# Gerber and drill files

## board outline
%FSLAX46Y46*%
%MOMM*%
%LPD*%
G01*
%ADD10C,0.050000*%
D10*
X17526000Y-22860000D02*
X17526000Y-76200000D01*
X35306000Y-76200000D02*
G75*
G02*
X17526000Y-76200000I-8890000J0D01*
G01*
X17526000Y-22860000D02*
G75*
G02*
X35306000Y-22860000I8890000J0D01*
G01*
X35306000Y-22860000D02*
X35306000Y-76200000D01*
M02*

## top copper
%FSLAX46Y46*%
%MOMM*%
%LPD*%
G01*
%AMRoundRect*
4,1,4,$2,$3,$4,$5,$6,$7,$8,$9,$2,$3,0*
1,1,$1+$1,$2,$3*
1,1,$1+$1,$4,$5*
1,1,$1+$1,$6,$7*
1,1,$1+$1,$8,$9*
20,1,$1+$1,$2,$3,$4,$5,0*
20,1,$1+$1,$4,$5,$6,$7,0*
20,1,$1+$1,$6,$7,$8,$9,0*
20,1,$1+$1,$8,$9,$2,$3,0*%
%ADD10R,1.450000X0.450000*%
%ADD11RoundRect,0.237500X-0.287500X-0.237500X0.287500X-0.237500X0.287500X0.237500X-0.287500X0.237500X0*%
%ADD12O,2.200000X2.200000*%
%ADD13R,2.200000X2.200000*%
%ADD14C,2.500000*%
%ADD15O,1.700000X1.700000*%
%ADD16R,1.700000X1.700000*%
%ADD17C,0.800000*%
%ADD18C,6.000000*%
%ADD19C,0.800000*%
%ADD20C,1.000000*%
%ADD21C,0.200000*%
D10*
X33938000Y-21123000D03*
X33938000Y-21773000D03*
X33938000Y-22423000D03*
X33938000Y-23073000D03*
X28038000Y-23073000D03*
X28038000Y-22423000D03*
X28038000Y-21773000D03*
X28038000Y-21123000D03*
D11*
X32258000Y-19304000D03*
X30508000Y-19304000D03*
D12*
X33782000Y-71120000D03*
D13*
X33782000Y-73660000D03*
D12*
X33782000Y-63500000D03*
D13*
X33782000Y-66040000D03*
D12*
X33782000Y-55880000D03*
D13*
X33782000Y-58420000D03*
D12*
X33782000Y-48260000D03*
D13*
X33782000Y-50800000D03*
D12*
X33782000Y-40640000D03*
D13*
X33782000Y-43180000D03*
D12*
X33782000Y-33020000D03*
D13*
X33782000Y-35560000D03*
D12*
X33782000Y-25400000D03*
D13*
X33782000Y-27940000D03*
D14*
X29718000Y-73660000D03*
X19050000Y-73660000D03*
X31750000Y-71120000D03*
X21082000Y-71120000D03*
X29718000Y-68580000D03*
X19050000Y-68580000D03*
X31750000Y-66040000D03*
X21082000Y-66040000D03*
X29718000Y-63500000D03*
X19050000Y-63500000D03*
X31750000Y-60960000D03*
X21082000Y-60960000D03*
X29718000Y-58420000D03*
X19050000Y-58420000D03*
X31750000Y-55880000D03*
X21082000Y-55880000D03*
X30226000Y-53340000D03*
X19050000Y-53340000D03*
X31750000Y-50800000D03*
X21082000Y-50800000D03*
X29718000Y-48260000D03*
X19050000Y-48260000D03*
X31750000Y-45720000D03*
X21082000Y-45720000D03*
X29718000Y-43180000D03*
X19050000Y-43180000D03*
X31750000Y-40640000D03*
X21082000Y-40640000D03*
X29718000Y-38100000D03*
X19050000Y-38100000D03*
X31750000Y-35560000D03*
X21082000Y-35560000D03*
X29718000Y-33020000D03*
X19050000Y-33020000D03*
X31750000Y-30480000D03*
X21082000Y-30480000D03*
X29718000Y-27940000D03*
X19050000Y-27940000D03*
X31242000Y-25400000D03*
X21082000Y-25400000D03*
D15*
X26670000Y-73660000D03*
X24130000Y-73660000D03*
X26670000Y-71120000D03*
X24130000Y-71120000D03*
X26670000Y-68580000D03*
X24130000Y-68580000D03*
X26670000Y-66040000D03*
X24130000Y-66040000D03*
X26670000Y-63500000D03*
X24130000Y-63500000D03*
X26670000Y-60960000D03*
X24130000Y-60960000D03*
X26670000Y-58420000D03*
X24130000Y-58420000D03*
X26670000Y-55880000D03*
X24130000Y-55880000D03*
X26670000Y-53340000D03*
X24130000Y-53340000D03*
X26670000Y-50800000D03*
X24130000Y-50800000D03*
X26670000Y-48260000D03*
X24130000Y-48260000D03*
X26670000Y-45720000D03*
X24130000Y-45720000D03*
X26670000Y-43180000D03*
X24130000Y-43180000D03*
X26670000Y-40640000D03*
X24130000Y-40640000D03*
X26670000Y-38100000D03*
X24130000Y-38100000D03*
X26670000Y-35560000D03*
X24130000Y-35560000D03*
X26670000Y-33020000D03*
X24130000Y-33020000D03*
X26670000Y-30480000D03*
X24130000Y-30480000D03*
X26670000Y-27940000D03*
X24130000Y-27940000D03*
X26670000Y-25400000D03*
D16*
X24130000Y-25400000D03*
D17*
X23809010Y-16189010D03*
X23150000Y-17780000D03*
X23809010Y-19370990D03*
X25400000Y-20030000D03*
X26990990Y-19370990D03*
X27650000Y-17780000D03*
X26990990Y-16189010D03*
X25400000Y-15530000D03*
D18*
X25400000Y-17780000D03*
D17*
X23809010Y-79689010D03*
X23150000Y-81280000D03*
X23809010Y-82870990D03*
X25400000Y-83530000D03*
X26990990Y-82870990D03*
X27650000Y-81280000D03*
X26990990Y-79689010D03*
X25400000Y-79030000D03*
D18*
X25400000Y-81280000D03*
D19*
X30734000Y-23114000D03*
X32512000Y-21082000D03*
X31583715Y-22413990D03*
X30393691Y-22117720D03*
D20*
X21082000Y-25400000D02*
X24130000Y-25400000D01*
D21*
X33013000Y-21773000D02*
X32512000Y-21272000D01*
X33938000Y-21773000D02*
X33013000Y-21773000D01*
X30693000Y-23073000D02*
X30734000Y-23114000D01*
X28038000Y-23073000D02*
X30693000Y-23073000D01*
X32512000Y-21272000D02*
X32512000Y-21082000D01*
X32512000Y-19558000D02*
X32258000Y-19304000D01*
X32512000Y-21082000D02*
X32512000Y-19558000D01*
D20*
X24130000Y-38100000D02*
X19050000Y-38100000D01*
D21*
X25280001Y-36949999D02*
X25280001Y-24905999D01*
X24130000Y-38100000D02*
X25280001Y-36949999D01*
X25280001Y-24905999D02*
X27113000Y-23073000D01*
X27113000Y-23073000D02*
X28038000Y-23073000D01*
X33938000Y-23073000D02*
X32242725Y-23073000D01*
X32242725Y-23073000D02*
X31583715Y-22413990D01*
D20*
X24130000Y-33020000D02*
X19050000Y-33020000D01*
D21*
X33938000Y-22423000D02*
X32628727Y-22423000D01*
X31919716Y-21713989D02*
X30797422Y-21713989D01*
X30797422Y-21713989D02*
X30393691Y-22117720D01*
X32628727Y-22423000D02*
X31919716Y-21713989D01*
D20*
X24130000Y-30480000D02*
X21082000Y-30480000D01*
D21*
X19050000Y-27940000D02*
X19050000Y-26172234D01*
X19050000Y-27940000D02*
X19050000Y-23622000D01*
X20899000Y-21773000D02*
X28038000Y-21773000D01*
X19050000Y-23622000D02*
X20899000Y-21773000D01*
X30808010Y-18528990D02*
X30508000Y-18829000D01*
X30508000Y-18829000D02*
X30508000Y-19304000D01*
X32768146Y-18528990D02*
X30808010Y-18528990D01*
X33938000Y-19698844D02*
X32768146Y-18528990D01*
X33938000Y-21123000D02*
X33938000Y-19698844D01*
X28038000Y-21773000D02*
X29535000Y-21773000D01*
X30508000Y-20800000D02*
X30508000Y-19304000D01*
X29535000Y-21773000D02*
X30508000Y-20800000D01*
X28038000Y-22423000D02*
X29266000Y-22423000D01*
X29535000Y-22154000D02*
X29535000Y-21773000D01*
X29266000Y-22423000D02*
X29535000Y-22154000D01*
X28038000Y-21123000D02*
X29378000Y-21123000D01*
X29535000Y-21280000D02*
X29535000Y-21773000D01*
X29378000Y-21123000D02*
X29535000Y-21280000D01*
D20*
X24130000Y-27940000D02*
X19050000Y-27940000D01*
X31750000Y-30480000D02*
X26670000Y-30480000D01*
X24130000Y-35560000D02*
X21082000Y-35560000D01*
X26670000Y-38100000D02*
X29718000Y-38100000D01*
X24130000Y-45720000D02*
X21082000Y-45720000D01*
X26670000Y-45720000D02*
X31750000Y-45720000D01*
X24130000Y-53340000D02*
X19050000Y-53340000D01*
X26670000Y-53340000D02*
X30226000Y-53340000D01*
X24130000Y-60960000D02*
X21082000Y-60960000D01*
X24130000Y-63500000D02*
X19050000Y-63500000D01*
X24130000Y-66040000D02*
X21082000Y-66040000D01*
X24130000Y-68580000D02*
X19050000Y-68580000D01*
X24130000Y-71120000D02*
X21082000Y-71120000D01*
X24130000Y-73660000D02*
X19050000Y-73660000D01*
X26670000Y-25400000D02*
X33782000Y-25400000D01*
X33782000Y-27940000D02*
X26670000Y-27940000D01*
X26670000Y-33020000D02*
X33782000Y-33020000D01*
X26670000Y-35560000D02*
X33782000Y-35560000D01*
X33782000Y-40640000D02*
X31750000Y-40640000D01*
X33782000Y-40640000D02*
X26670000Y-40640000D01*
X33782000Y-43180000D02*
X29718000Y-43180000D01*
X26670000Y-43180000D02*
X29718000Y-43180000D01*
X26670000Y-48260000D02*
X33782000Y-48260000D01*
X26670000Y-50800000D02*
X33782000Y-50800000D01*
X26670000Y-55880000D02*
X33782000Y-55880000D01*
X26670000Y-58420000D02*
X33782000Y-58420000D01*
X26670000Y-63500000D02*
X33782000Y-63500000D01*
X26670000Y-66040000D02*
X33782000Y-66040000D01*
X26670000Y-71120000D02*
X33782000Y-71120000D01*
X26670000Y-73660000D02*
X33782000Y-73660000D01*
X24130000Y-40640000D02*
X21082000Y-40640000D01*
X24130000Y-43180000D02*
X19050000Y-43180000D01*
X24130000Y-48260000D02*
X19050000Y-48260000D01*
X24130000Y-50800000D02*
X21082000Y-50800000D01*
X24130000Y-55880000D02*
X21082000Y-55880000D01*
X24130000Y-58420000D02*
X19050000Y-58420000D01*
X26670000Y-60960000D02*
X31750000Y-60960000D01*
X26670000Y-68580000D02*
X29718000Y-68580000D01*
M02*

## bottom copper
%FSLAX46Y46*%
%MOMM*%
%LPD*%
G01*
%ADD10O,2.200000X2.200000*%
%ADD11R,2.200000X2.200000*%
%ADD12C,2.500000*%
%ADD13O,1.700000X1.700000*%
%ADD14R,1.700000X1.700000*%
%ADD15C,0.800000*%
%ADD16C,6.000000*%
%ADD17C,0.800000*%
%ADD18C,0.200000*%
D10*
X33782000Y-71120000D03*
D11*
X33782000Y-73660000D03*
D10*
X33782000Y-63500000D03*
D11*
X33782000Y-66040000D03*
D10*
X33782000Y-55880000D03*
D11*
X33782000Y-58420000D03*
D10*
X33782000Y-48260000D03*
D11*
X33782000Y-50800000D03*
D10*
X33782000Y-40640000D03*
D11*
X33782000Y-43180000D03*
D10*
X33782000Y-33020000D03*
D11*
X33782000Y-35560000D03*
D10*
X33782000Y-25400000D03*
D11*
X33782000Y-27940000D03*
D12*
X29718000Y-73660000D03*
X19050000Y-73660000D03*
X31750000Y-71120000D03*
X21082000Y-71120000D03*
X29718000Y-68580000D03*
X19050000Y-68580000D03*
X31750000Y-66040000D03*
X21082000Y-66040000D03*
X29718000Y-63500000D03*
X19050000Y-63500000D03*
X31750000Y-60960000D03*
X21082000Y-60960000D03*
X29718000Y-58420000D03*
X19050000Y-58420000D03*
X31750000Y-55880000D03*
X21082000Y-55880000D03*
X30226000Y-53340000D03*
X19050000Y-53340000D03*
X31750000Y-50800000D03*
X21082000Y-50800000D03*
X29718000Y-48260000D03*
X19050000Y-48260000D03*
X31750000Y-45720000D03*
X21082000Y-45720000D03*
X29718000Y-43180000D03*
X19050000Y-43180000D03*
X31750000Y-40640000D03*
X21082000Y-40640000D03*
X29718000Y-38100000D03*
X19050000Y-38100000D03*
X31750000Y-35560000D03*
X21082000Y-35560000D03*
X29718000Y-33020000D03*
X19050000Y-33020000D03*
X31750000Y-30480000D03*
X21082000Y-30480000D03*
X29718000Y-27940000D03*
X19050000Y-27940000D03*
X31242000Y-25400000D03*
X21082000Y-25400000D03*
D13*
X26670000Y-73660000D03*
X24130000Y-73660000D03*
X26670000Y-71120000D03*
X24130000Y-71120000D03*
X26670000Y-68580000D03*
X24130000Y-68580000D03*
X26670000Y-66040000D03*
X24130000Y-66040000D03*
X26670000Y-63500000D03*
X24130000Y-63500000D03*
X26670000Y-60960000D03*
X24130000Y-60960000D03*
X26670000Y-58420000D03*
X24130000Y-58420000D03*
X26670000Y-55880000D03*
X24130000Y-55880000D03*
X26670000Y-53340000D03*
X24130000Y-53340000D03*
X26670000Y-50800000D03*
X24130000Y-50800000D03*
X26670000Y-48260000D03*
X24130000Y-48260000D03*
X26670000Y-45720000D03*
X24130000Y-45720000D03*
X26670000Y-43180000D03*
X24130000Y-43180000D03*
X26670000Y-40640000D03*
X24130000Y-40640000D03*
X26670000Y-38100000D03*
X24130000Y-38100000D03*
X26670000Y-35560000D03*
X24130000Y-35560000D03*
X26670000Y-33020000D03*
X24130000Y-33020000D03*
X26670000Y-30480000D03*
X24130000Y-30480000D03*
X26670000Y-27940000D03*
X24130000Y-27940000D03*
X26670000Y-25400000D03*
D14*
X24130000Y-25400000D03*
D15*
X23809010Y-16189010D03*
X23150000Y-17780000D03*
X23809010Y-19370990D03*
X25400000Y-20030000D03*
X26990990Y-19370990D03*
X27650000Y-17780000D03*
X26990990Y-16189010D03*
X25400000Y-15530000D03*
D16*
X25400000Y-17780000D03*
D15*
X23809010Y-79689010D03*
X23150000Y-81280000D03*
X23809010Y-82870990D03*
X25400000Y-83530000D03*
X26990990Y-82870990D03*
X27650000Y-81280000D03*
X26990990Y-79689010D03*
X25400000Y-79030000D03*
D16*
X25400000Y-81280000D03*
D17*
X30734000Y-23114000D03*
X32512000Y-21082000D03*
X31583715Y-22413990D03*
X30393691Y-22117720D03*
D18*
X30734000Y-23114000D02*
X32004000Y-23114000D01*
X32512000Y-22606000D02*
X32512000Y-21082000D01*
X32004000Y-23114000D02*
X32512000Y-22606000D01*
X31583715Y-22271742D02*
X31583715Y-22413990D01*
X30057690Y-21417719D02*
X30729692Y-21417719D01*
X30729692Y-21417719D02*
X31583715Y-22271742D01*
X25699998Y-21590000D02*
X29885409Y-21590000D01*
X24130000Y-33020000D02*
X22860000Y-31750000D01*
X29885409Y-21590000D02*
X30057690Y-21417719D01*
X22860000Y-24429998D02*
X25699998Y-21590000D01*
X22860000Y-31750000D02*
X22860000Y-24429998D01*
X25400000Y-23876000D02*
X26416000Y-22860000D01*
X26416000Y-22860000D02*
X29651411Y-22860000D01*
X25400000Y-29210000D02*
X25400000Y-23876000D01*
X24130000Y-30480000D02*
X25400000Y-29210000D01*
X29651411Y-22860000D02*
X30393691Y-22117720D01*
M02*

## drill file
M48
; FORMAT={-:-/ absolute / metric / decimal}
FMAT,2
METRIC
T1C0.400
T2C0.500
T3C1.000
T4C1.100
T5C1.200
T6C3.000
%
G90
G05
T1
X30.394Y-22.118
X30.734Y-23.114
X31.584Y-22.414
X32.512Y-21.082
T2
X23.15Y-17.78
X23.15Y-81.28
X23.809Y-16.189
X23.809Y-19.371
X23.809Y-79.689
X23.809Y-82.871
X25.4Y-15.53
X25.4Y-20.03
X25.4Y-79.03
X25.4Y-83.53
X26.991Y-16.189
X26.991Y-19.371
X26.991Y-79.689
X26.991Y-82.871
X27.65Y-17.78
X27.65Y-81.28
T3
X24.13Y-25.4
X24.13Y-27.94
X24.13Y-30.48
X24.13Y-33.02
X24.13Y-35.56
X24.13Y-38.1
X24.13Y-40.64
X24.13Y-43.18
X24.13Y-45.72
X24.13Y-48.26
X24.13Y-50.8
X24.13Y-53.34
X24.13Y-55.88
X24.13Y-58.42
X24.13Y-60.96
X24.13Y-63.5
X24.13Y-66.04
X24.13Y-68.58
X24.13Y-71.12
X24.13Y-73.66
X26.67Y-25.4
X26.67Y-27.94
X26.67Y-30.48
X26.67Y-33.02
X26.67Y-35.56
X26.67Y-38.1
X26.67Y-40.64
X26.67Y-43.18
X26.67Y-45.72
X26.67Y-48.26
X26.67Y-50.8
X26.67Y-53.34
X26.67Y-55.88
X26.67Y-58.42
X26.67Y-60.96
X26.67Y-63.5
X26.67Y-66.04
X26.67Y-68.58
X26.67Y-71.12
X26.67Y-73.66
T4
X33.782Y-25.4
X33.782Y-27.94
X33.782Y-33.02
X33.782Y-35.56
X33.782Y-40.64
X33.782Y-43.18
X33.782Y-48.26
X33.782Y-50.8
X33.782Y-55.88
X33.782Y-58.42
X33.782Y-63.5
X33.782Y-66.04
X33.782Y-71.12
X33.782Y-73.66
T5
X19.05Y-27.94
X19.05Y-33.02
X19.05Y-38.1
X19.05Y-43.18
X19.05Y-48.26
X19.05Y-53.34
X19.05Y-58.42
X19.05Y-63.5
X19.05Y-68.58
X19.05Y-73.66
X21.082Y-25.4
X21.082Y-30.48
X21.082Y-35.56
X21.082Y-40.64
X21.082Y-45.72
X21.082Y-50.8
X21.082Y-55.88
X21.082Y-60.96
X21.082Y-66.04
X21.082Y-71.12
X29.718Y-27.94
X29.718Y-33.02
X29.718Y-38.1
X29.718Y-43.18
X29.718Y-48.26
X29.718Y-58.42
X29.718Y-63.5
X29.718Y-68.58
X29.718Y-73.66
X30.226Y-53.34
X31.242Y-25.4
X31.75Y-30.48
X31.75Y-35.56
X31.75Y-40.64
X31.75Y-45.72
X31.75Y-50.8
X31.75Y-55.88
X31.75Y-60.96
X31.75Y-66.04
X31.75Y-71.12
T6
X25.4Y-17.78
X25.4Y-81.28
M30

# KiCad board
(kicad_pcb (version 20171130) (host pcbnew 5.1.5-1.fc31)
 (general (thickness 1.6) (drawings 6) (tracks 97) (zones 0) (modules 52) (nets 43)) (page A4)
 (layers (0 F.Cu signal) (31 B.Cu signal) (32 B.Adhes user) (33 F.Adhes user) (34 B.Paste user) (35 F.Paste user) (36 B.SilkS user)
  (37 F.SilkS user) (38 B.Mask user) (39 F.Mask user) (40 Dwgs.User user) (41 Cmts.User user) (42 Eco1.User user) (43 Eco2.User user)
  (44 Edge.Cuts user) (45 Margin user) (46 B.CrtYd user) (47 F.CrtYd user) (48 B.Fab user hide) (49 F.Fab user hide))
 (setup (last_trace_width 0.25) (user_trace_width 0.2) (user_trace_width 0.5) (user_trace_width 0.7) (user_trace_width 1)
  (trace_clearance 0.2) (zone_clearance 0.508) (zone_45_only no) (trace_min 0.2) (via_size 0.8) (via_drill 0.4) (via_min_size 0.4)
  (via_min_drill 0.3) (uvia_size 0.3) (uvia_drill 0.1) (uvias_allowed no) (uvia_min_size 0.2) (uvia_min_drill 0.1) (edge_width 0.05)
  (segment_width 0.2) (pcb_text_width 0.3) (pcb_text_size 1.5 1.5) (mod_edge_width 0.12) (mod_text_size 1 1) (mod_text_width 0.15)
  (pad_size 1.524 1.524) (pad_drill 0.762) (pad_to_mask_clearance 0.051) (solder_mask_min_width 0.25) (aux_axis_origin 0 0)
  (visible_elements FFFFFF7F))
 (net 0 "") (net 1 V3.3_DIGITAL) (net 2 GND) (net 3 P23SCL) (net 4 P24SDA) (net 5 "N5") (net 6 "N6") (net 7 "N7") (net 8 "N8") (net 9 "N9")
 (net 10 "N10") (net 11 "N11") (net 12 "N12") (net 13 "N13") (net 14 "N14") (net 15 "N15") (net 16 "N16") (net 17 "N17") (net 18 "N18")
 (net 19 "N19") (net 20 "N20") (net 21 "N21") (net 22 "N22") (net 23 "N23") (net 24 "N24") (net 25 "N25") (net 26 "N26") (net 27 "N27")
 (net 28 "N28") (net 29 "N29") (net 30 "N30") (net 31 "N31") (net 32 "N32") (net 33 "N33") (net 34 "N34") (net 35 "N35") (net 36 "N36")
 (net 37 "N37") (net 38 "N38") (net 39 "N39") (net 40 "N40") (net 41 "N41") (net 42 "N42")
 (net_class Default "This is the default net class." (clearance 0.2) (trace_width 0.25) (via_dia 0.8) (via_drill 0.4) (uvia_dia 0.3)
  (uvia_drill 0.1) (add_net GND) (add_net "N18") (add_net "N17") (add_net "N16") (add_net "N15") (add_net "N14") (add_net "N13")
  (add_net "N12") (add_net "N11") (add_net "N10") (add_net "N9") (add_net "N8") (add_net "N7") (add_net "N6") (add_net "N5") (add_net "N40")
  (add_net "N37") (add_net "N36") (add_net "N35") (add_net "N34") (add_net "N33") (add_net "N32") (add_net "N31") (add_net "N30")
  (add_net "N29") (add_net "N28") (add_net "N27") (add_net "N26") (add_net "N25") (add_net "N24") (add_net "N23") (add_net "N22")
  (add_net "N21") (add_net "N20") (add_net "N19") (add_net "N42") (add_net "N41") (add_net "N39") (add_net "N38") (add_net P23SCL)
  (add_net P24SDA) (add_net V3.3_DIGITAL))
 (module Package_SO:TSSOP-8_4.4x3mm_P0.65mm (layer F.Cu) (at 30.988 22.098)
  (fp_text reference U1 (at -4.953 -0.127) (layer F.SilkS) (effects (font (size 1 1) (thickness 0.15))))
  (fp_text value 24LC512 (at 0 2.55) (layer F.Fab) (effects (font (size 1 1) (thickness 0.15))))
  (pad 8 smd rect (at 2.95 -0.975) (size 1.45 0.45) (layers F.Cu F.Paste F.Mask) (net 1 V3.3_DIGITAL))
  (pad 7 smd rect (at 2.95 -0.325) (size 1.45 0.45) (layers F.Cu F.Paste F.Mask) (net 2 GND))
  (pad 6 smd rect (at 2.95 0.325) (size 1.45 0.45) (layers F.Cu F.Paste F.Mask) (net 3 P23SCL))
  (pad 5 smd rect (at 2.95 0.975) (size 1.45 0.45) (layers F.Cu F.Paste F.Mask) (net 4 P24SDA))
  (pad 4 smd rect (at -2.95 0.975) (size 1.45 0.45) (layers F.Cu F.Paste F.Mask) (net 2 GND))
  (pad 3 smd rect (at -2.95 0.325) (size 1.45 0.45) (layers F.Cu F.Paste F.Mask) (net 1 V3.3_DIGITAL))
  (pad 2 smd rect (at -2.95 -0.325) (size 1.45 0.45) (layers F.Cu F.Paste F.Mask) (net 1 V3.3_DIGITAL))
  (pad 1 smd rect (at -2.95 -0.975) (size 1.45 0.45) (layers F.Cu F.Paste F.Mask) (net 1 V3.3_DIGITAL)))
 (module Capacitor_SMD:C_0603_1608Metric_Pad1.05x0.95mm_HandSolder (layer F.Cu) (at 31.383 19.304)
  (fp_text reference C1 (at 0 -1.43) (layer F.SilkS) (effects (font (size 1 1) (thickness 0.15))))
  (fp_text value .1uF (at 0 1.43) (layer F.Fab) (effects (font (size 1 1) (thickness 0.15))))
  (pad 2 smd roundrect (at 0.875 0) (size 1.05 0.95) (layers F.Cu F.Paste F.Mask) (roundrect_rratio 0.25) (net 2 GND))
  (pad 1 smd roundrect (at -0.875 0) (size 1.05 0.95) (layers F.Cu F.Paste F.Mask) (roundrect_rratio 0.25) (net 1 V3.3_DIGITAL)))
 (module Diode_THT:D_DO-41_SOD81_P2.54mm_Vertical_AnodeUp (layer B.Cu) (at 33.782 73.66 90)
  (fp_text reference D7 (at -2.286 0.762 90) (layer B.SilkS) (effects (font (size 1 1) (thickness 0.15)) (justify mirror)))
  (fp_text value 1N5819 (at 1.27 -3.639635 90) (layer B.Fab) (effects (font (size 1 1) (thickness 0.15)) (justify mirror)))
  (pad 2 thru_hole oval (at 2.54 0 90) (size 2.2 2.2) (drill 1.1) (layers *.Cu *.Mask) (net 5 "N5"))
  (pad 1 thru_hole rect (at 0 0 90) (size 2.2 2.2) (drill 1.1) (layers *.Cu *.Mask) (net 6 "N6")))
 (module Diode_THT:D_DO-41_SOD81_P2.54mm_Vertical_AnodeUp (layer B.Cu) (at 33.782 66.04 90)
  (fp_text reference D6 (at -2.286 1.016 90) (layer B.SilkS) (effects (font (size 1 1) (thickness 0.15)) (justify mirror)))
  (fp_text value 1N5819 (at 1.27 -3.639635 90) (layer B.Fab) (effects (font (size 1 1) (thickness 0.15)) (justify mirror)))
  (pad 2 thru_hole oval (at 2.54 0 90) (size 2.2 2.2) (drill 1.1) (layers *.Cu *.Mask) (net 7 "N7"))
  (pad 1 thru_hole rect (at 0 0 90) (size 2.2 2.2) (drill 1.1) (layers *.Cu *.Mask) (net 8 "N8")))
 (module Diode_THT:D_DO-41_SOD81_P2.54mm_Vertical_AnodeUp (layer B.Cu) (at 33.782 58.42 90)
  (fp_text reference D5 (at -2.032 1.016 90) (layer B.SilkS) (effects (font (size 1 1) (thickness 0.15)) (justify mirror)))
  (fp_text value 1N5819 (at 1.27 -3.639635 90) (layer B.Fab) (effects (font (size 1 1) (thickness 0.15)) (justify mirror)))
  (pad 2 thru_hole oval (at 2.54 0 90) (size 2.2 2.2) (drill 1.1) (layers *.Cu *.Mask) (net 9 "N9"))
  (pad 1 thru_hole rect (at 0 0 90) (size 2.2 2.2) (drill 1.1) (layers *.Cu *.Mask) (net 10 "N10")))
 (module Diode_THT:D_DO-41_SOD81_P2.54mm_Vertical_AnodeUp (layer B.Cu) (at 33.782 50.8 90)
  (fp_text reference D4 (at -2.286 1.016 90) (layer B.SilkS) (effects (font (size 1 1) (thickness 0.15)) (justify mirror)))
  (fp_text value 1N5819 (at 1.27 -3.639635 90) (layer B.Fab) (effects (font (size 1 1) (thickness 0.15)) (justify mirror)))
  (pad 2 thru_hole oval (at 2.54 0 90) (size 2.2 2.2) (drill 1.1) (layers *.Cu *.Mask) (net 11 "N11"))
  (pad 1 thru_hole rect (at 0 0 90) (size 2.2 2.2) (drill 1.1) (layers *.Cu *.Mask) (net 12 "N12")))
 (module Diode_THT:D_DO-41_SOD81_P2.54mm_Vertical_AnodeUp (layer B.Cu) (at 33.782 43.18 90)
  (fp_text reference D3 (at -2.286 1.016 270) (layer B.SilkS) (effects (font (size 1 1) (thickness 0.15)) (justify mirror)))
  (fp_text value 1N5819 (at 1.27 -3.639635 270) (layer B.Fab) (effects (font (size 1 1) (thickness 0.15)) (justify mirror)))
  (pad 2 thru_hole oval (at 2.54 0 90) (size 2.2 2.2) (drill 1.1) (layers *.Cu *.Mask) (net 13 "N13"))
  (pad 1 thru_hole rect (at 0 0 90) (size 2.2 2.2) (drill 1.1) (layers *.Cu *.Mask) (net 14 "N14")))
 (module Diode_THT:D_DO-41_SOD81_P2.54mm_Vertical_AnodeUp (layer B.Cu) (at 33.782 35.56 90)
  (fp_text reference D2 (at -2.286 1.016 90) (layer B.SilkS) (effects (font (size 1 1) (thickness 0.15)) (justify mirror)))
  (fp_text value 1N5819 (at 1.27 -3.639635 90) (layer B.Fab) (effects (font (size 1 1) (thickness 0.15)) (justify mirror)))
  (pad 2 thru_hole oval (at 2.54 0 90) (size 2.2 2.2) (drill 1.1) (layers *.Cu *.Mask) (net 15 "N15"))
  (pad 1 thru_hole rect (at 0 0 90) (size 2.2 2.2) (drill 1.1) (layers *.Cu *.Mask) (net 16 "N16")))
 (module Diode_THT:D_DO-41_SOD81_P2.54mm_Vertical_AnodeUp (layer B.Cu) (at 33.782 27.94 90)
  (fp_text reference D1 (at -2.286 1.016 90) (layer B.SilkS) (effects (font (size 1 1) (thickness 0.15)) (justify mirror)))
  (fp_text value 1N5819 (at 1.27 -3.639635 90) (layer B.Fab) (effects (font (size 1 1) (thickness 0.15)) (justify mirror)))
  (pad 2 thru_hole oval (at 2.54 0 90) (size 2.2 2.2) (drill 1.1) (layers *.Cu *.Mask) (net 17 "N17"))
  (pad 1 thru_hole rect (at 0 0 90) (size 2.2 2.2) (drill 1.1) (layers *.Cu *.Mask) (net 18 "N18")))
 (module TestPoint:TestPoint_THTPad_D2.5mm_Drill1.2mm (layer F.Cu) (at 29.718 73.66 270)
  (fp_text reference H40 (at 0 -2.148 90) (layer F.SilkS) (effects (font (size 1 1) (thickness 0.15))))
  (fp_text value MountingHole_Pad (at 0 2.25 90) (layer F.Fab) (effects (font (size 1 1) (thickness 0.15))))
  (pad 1 thru_hole circle (at 0 0 270) (size 2.5 2.5) (drill 1.2) (layers *.Cu *.Mask) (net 6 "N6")))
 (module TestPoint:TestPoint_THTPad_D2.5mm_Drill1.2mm (layer F.Cu) (at 19.05 73.66 270)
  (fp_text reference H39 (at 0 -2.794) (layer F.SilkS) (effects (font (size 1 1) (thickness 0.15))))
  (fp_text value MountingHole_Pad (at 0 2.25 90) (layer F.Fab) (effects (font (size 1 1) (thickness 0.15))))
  (pad 1 thru_hole circle (at 0 0 270) (size 2.5 2.5) (drill 1.2) (layers *.Cu *.Mask) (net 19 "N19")))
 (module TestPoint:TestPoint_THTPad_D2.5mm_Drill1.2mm (layer F.Cu) (at 31.75 71.12 90)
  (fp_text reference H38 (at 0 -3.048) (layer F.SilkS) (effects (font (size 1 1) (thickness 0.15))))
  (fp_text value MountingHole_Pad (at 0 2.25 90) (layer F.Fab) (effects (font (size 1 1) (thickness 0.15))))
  (pad 1 thru_hole circle (at 0 0 90) (size 2.5 2.5) (drill 1.2) (layers *.Cu *.Mask) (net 5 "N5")))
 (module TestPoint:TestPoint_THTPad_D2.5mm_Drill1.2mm (layer F.Cu) (at 21.082 71.12 90)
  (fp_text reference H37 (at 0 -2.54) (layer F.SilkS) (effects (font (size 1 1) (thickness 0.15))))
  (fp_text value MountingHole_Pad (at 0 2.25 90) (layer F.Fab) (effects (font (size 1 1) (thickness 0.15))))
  (pad 1 thru_hole circle (at 0 0 90) (size 2.5 2.5) (drill 1.2) (layers *.Cu *.Mask) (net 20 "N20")))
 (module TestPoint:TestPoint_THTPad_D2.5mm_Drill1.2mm (layer F.Cu) (at 29.718 68.58 270)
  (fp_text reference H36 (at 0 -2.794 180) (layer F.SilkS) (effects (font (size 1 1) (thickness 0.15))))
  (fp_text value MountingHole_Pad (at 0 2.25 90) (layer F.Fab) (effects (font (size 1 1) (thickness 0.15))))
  (pad 1 thru_hole circle (at 0 0 270) (size 2.5 2.5) (drill 1.2) (layers *.Cu *.Mask) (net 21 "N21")))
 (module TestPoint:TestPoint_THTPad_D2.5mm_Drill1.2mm (layer F.Cu) (at 19.05 68.58 270)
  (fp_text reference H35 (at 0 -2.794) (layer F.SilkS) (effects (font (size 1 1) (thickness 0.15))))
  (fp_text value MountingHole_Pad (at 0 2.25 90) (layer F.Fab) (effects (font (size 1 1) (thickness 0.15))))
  (pad 1 thru_hole circle (at 0 0 270) (size 2.5 2.5) (drill 1.2) (layers *.Cu *.Mask) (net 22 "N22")))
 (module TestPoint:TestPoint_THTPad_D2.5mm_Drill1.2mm (layer F.Cu) (at 31.75 66.04 90)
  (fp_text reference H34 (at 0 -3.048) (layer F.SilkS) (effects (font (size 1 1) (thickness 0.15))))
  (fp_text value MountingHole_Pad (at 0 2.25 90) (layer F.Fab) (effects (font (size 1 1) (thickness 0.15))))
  (pad 1 thru_hole circle (at 0 0 90) (size 2.5 2.5) (drill 1.2) (layers *.Cu *.Mask) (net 8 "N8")))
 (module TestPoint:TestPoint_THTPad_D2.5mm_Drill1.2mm (layer F.Cu) (at 21.082 66.04 90)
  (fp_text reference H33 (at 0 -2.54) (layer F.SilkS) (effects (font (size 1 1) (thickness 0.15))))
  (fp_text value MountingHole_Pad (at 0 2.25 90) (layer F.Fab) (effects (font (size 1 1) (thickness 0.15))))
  (pad 1 thru_hole circle (at 0 0 90) (size 2.5 2.5) (drill 1.2) (layers *.Cu *.Mask) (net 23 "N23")))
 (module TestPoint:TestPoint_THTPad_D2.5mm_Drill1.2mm (layer F.Cu) (at 29.718 63.5 270)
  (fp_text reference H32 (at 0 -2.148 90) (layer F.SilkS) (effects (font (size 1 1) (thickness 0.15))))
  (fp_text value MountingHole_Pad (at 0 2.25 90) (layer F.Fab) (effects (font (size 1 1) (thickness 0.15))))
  (pad 1 thru_hole circle (at 0 0 270) (size 2.5 2.5) (drill 1.2) (layers *.Cu *.Mask) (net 7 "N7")))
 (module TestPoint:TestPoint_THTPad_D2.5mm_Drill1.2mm (layer F.Cu) (at 19.05 63.5 270)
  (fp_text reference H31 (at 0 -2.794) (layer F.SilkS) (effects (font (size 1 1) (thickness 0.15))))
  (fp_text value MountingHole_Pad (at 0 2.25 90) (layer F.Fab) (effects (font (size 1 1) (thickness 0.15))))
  (pad 1 thru_hole circle (at 0 0 270) (size 2.5 2.5) (drill 1.2) (layers *.Cu *.Mask) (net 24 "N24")))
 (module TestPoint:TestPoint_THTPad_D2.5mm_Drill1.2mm (layer F.Cu) (at 31.75 60.96 90)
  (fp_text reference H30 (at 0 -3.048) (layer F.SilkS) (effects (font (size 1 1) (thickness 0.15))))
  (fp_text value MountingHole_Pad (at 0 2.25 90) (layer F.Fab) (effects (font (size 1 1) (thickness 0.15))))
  (pad 1 thru_hole circle (at 0 0 90) (size 2.5 2.5) (drill 1.2) (layers *.Cu *.Mask) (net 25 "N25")))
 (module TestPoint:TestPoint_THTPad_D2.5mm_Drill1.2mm (layer F.Cu) (at 21.082 60.96 90)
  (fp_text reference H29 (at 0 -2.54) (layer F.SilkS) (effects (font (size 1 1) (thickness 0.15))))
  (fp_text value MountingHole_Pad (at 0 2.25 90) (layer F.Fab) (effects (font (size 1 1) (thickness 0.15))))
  (pad 1 thru_hole circle (at 0 0 90) (size 2.5 2.5) (drill 1.2) (layers *.Cu *.Mask) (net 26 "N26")))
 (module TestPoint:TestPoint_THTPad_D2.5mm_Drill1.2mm (layer F.Cu) (at 29.718 58.42 270)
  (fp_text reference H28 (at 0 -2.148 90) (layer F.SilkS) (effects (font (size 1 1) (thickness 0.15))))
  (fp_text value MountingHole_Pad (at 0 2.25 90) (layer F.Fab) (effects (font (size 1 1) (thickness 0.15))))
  (pad 1 thru_hole circle (at 0 0 270) (size 2.5 2.5) (drill 1.2) (layers *.Cu *.Mask) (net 10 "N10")))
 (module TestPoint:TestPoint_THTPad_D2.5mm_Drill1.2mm (layer F.Cu) (at 19.05 58.42 270)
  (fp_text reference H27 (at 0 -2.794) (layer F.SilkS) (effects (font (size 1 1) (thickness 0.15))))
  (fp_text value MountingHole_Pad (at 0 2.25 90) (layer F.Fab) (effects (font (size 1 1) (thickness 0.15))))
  (pad 1 thru_hole circle (at 0 0 270) (size 2.5 2.5) (drill 1.2) (layers *.Cu *.Mask) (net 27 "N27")))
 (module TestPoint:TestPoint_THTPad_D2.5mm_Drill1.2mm (layer F.Cu) (at 31.75 55.88 90)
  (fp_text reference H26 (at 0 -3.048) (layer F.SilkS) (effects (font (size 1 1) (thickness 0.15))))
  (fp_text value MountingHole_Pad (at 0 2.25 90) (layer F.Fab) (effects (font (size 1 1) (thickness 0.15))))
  (pad 1 thru_hole circle (at 0 0 90) (size 2.5 2.5) (drill 1.2) (layers *.Cu *.Mask) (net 9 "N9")))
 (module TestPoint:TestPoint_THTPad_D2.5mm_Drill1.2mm (layer F.Cu) (at 21.082 55.88 90)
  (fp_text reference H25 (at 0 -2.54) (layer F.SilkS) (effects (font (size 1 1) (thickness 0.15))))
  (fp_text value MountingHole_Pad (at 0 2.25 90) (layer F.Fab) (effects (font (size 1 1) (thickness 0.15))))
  (pad 1 thru_hole circle (at 0 0 90) (size 2.5 2.5) (drill 1.2) (layers *.Cu *.Mask) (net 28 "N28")))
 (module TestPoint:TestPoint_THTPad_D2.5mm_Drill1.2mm (layer F.Cu) (at 30.226 53.34 270)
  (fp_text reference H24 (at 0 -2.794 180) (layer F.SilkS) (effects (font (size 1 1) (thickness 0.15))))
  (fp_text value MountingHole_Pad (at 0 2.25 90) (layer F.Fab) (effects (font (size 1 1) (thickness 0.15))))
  (pad 1 thru_hole circle (at 0 0 270) (size 2.5 2.5) (drill 1.2) (layers *.Cu *.Mask) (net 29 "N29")))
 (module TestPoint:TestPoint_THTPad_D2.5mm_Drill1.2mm (layer F.Cu) (at 19.05 53.34 270)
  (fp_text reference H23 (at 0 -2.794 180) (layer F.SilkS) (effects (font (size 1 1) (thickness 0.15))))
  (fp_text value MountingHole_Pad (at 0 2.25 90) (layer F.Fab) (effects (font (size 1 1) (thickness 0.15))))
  (pad 1 thru_hole circle (at 0 0 270) (size 2.5 2.5) (drill 1.2) (layers *.Cu *.Mask) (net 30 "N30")))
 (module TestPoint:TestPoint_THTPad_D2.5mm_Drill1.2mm (layer F.Cu) (at 31.75 50.8 90)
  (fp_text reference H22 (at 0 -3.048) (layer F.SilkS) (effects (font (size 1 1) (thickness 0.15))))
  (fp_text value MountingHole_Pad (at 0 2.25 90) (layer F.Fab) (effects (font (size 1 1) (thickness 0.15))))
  (pad 1 thru_hole circle (at 0 0 90) (size 2.5 2.5) (drill 1.2) (layers *.Cu *.Mask) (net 12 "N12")))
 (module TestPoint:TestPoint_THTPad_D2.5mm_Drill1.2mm (layer F.Cu) (at 21.082 50.8 90)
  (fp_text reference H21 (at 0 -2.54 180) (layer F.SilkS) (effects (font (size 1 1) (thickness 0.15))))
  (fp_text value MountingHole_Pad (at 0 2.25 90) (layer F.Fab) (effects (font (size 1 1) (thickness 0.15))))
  (pad 1 thru_hole circle (at 0 0 90) (size 2.5 2.5) (drill 1.2) (layers *.Cu *.Mask) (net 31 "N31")))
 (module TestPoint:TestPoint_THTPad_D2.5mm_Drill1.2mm (layer F.Cu) (at 29.718 48.26 270)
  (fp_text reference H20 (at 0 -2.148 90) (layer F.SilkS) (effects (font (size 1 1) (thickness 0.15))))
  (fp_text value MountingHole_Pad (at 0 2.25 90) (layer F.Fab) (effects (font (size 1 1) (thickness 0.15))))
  (pad 1 thru_hole circle (at 0 0 270) (size 2.5 2.5) (drill 1.2) (layers *.Cu *.Mask) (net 11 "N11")))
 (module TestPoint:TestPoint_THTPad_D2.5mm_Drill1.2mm (layer F.Cu) (at 19.05 48.26 270)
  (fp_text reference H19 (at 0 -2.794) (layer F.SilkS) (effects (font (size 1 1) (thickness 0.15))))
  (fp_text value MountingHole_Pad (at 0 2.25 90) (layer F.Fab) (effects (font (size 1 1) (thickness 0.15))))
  (pad 1 thru_hole circle (at 0 0 270) (size 2.5 2.5) (drill 1.2) (layers *.Cu *.Mask) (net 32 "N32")))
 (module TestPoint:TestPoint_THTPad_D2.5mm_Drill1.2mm (layer F.Cu) (at 31.75 45.72 90)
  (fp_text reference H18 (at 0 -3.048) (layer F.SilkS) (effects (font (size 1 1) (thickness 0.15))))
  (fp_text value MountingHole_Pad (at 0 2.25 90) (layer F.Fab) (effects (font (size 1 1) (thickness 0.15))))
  (pad 1 thru_hole circle (at 0 0 90) (size 2.5 2.5) (drill 1.2) (layers *.Cu *.Mask) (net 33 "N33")))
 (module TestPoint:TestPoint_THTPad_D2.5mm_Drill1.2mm (layer F.Cu) (at 21.082 45.72 90)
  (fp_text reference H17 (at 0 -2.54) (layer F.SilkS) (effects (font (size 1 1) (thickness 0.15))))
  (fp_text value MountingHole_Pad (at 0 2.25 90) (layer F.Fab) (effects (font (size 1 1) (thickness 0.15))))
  (pad 1 thru_hole circle (at 0 0 90) (size 2.5 2.5) (drill 1.2) (layers *.Cu *.Mask) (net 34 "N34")))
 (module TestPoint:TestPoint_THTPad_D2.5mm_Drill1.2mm (layer F.Cu) (at 29.718 43.18 270)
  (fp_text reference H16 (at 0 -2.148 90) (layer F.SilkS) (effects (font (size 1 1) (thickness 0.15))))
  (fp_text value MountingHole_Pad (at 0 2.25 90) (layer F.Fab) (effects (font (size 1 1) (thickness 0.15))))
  (pad 1 thru_hole circle (at 0 0 270) (size 2.5 2.5) (drill 1.2) (layers *.Cu *.Mask) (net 14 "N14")))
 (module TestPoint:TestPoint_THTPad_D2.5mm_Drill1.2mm (layer F.Cu) (at 19.05 43.18 270)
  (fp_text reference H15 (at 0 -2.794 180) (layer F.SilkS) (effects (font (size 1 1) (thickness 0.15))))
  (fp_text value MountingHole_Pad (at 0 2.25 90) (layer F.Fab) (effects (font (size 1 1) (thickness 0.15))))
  (pad 1 thru_hole circle (at 0 0 270) (size 2.5 2.5) (drill 1.2) (layers *.Cu *.Mask) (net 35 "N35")))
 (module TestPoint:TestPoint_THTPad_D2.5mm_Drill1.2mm (layer F.Cu) (at 31.75 40.64 90)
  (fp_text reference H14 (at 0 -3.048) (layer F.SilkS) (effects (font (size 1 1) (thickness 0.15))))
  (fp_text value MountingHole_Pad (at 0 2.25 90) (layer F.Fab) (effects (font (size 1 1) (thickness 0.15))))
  (pad 1 thru_hole circle (at 0 0 90) (size 2.5 2.5) (drill 1.2) (layers *.Cu *.Mask) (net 13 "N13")))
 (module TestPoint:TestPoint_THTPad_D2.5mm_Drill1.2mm (layer F.Cu) (at 21.082 40.64 90)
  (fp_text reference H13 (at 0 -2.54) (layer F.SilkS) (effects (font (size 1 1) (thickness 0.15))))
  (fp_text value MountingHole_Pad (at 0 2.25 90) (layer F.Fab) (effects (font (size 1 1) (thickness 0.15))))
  (pad 1 thru_hole circle (at 0 0 90) (size 2.5 2.5) (drill 1.2) (layers *.Cu *.Mask) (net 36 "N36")))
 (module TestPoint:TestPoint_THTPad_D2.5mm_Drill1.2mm (layer F.Cu) (at 29.718 38.1 270)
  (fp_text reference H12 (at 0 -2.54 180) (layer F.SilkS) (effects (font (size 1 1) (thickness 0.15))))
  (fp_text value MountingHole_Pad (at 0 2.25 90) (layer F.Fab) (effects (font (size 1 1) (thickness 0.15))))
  (pad 1 thru_hole circle (at 0 0 270) (size 2.5 2.5) (drill 1.2) (layers *.Cu *.Mask) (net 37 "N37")))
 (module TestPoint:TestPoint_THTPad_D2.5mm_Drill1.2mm (layer F.Cu) (at 19.05 38.1 270)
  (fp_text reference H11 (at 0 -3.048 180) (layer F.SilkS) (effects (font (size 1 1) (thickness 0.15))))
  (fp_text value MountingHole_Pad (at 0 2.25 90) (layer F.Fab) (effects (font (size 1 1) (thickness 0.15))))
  (pad 1 thru_hole circle (at 0 0 270) (size 2.5 2.5) (drill 1.2) (layers *.Cu *.Mask) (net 2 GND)))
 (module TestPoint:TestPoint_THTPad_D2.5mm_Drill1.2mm (layer F.Cu) (at 31.75 35.56 90)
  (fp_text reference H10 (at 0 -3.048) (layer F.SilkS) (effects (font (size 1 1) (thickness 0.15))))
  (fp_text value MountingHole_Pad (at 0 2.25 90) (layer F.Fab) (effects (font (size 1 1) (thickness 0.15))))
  (pad 1 thru_hole circle (at 0 0 90) (size 2.5 2.5) (drill 1.2) (layers *.Cu *.Mask) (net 16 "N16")))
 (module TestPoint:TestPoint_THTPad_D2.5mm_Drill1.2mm (layer F.Cu) (at 21.082 35.56 90)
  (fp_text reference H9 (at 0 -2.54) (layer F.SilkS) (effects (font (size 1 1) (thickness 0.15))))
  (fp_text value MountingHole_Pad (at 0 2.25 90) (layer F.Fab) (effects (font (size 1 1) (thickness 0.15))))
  (pad 1 thru_hole circle (at 0 0 90) (size 2.5 2.5) (drill 1.2) (layers *.Cu *.Mask) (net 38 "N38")))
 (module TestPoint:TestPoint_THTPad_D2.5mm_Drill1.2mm (layer F.Cu) (at 29.718 33.02 270)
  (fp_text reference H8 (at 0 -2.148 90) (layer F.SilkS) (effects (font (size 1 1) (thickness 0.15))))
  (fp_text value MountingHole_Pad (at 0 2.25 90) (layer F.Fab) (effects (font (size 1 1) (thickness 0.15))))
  (pad 1 thru_hole circle (at 0 0 270) (size 2.5 2.5) (drill 1.2) (layers *.Cu *.Mask) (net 15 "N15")))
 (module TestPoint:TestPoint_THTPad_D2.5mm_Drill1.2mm (layer F.Cu) (at 19.05 33.02 270)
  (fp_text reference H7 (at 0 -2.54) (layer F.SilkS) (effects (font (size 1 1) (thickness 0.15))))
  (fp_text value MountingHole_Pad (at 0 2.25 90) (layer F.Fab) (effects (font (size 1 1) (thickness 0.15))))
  (pad 1 thru_hole circle (at 0 0 270) (size 2.5 2.5) (drill 1.2) (layers *.Cu *.Mask) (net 4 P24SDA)))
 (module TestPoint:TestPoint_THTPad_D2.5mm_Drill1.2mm (layer F.Cu) (at 31.75 30.48 90)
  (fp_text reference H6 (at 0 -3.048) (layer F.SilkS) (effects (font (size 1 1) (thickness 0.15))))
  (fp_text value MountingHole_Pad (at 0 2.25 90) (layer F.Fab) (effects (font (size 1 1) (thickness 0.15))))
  (pad 1 thru_hole circle (at 0 0 90) (size 2.5 2.5) (drill 1.2) (layers *.Cu *.Mask) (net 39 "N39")))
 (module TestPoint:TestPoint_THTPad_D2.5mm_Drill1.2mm (layer F.Cu) (at 21.082 30.48 90)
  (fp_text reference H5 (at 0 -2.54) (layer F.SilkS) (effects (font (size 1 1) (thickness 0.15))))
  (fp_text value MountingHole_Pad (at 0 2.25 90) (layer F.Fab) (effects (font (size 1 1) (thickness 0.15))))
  (pad 1 thru_hole circle (at 0 0 90) (size 2.5 2.5) (drill 1.2) (layers *.Cu *.Mask) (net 3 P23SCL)))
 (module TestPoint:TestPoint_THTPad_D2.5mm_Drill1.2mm (layer F.Cu) (at 29.718 27.94 270)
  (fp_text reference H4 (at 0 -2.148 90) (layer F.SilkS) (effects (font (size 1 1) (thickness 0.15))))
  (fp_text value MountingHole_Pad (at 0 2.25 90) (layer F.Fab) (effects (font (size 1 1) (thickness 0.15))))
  (pad 1 thru_hole circle (at 0 0 270) (size 2.5 2.5) (drill 1.2) (layers *.Cu *.Mask) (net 18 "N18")))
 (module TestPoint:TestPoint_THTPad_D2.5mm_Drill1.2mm (layer F.Cu) (at 19.05 27.94 270)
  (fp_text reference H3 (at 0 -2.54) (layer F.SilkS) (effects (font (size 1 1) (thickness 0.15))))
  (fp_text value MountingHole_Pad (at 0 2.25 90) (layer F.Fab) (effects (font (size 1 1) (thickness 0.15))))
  (pad 1 thru_hole circle (at 0 0 270) (size 2.5 2.5) (drill 1.2) (layers *.Cu *.Mask) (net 1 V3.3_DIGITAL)))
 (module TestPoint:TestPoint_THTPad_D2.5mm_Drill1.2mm (layer F.Cu) (at 31.242 25.4 90)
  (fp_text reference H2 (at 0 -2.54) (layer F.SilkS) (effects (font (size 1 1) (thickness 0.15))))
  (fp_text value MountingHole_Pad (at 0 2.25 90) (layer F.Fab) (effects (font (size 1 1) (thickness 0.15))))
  (pad 1 thru_hole circle (at 0 0 90) (size 2.5 2.5) (drill 1.2) (layers *.Cu *.Mask) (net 17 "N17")))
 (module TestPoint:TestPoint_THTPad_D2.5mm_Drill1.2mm (layer F.Cu) (at 21.082 25.4 90)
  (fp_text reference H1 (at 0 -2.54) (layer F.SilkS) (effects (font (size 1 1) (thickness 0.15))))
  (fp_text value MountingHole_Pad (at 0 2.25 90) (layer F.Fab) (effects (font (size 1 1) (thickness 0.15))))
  (pad 1 thru_hole circle (at 0 0 90) (size 2.5 2.5) (drill 1.2) (layers *.Cu *.Mask) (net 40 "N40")))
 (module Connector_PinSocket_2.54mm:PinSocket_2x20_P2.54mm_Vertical (layer B.Cu) (at 24.13 25.4 180)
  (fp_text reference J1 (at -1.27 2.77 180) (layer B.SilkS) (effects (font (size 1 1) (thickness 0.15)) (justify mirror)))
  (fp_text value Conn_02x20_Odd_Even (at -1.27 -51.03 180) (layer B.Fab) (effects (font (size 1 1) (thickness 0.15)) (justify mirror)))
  (pad 40 thru_hole oval (at -2.54 -48.26 180) (size 1.7 1.7) (drill 1) (layers *.Cu *.Mask) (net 6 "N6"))
  (pad 39 thru_hole oval (at 0 -48.26 180) (size 1.7 1.7) (drill 1) (layers *.Cu *.Mask) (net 19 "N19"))
  (pad 38 thru_hole oval (at -2.54 -45.72 180) (size 1.7 1.7) (drill 1) (layers *.Cu *.Mask) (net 5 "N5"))
  (pad 37 thru_hole oval (at 0 -45.72 180) (size 1.7 1.7) (drill 1) (layers *.Cu *.Mask) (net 20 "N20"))
  (pad 36 thru_hole oval (at -2.54 -43.18 180) (size 1.7 1.7) (drill 1) (layers *.Cu *.Mask) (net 21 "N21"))
  (pad 35 thru_hole oval (at 0 -43.18 180) (size 1.7 1.7) (drill 1) (layers *.Cu *.Mask) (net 22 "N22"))
  (pad 34 thru_hole oval (at -2.54 -40.64 180) (size 1.7 1.7) (drill 1) (layers *.Cu *.Mask) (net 8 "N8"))
  (pad 33 thru_hole oval (at 0 -40.64 180) (size 1.7 1.7) (drill 1) (layers *.Cu *.Mask) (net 23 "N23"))
  (pad 32 thru_hole oval (at -2.54 -38.1 180) (size 1.7 1.7) (drill 1) (layers *.Cu *.Mask) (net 7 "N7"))
  (pad 31 thru_hole oval (at 0 -38.1 180) (size 1.7 1.7) (drill 1) (layers *.Cu *.Mask) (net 24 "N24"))
  (pad 30 thru_hole oval (at -2.54 -35.56 180) (size 1.7 1.7) (drill 1) (layers *.Cu *.Mask) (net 25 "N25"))
  (pad 29 thru_hole oval (at 0 -35.56 180) (size 1.7 1.7) (drill 1) (layers *.Cu *.Mask) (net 26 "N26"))
  (pad 28 thru_hole oval (at -2.54 -33.02 180) (size 1.7 1.7) (drill 1) (layers *.Cu *.Mask) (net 10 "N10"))
  (pad 27 thru_hole oval (at 0 -33.02 180) (size 1.7 1.7) (drill 1) (layers *.Cu *.Mask) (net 27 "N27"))
  (pad 26 thru_hole oval (at -2.54 -30.48 180) (size 1.7 1.7) (drill 1) (layers *.Cu *.Mask) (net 9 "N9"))
  (pad 25 thru_hole oval (at 0 -30.48 180) (size 1.7 1.7) (drill 1) (layers *.Cu *.Mask) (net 28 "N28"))
  (pad 24 thru_hole oval (at -2.54 -27.94 180) (size 1.7 1.7) (drill 1) (layers *.Cu *.Mask) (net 29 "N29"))
  (pad 23 thru_hole oval (at 0 -27.94 180) (size 1.7 1.7) (drill 1) (layers *.Cu *.Mask) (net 30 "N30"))
  (pad 22 thru_hole oval (at -2.54 -25.4 180) (size 1.7 1.7) (drill 1) (layers *.Cu *.Mask) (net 12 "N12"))
  (pad 21 thru_hole oval (at 0 -25.4 180) (size 1.7 1.7) (drill 1) (layers *.Cu *.Mask) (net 31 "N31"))
  (pad 20 thru_hole oval (at -2.54 -22.86 180) (size 1.7 1.7) (drill 1) (layers *.Cu *.Mask) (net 11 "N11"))
  (pad 19 thru_hole oval (at 0 -22.86 180) (size 1.7 1.7) (drill 1) (layers *.Cu *.Mask) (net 32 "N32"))
  (pad 18 thru_hole oval (at -2.54 -20.32 180) (size 1.7 1.7) (drill 1) (layers *.Cu *.Mask) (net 33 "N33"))
  (pad 17 thru_hole oval (at 0 -20.32 180) (size 1.7 1.7) (drill 1) (layers *.Cu *.Mask) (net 34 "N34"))
  (pad 16 thru_hole oval (at -2.54 -17.78 180) (size 1.7 1.7) (drill 1) (layers *.Cu *.Mask) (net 14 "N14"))
  (pad 15 thru_hole oval (at 0 -17.78 180) (size 1.7 1.7) (drill 1) (layers *.Cu *.Mask) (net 35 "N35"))
  (pad 14 thru_hole oval (at -2.54 -15.24 180) (size 1.7 1.7) (drill 1) (layers *.Cu *.Mask) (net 13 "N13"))
  (pad 13 thru_hole oval (at 0 -15.24 180) (size 1.7 1.7) (drill 1) (layers *.Cu *.Mask) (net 36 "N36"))
  (pad 12 thru_hole oval (at -2.54 -12.7 180) (size 1.7 1.7) (drill 1) (layers *.Cu *.Mask) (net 37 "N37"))
  (pad 11 thru_hole oval (at 0 -12.7 180) (size 1.7 1.7) (drill 1) (layers *.Cu *.Mask) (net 2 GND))
  (pad 10 thru_hole oval (at -2.54 -10.16 180) (size 1.7 1.7) (drill 1) (layers *.Cu *.Mask) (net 16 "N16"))
  (pad 9 thru_hole oval (at 0 -10.16 180) (size 1.7 1.7) (drill 1) (layers *.Cu *.Mask) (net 38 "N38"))
  (pad 8 thru_hole oval (at -2.54 -7.62 180) (size 1.7 1.7) (drill 1) (layers *.Cu *.Mask) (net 15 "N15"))
  (pad 7 thru_hole oval (at 0 -7.62 180) (size 1.7 1.7) (drill 1) (layers *.Cu *.Mask) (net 4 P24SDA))
  (pad 6 thru_hole oval (at -2.54 -5.08 180) (size 1.7 1.7) (drill 1) (layers *.Cu *.Mask) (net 39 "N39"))
  (pad 5 thru_hole oval (at 0 -5.08 180) (size 1.7 1.7) (drill 1) (layers *.Cu *.Mask) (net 3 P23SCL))
  (pad 4 thru_hole oval (at -2.54 -2.54 180) (size 1.7 1.7) (drill 1) (layers *.Cu *.Mask) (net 18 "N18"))
  (pad 3 thru_hole oval (at 0 -2.54 180) (size 1.7 1.7) (drill 1) (layers *.Cu *.Mask) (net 1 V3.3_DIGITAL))
  (pad 2 thru_hole oval (at -2.54 0 180) (size 1.7 1.7) (drill 1) (layers *.Cu *.Mask) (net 17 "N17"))
  (pad 1 thru_hole rect (at 0 0 180) (size 1.7 1.7) (drill 1) (layers *.Cu *.Mask) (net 40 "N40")))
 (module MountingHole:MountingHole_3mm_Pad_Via (layer F.Cu) (at 25.4 17.78 90)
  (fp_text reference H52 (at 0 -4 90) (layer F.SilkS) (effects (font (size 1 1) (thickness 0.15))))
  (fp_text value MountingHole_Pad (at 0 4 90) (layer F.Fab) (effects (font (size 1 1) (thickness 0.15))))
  (pad 1 thru_hole circle (at 1.59099 -1.59099 90) (size 0.8 0.8) (drill 0.5) (layers *.Cu *.Mask) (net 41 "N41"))
  (pad 1 thru_hole circle (at 0 -2.25 90) (size 0.8 0.8) (drill 0.5) (layers *.Cu *.Mask) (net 41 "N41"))
  (pad 1 thru_hole circle (at -1.59099 -1.59099 90) (size 0.8 0.8) (drill 0.5) (layers *.Cu *.Mask) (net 41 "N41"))
  (pad 1 thru_hole circle (at -2.25 0 90) (size 0.8 0.8) (drill 0.5) (layers *.Cu *.Mask) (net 41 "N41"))
  (pad 1 thru_hole circle (at -1.59099 1.59099 90) (size 0.8 0.8) (drill 0.5) (layers *.Cu *.Mask) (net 41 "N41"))
  (pad 1 thru_hole circle (at 0 2.25 90) (size 0.8 0.8) (drill 0.5) (layers *.Cu *.Mask) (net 41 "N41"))
  (pad 1 thru_hole circle (at 1.59099 1.59099 90) (size 0.8 0.8) (drill 0.5) (layers *.Cu *.Mask) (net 41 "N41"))
  (pad 1 thru_hole circle (at 2.25 0 90) (size 0.8 0.8) (drill 0.5) (layers *.Cu *.Mask) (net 41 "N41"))
  (pad 1 thru_hole circle (at 0 0 90) (size 6 6) (drill 3) (layers *.Cu *.Mask) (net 41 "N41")))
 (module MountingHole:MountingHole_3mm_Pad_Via (layer F.Cu) (at 25.4 81.28 90)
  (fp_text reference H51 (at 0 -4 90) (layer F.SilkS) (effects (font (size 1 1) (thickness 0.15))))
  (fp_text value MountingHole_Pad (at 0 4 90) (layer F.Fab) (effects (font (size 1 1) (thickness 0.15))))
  (pad 1 thru_hole circle (at 1.59099 -1.59099 90) (size 0.8 0.8) (drill 0.5) (layers *.Cu *.Mask) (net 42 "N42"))
  (pad 1 thru_hole circle (at 0 -2.25 90) (size 0.8 0.8) (drill 0.5) (layers *.Cu *.Mask) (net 42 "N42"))
  (pad 1 thru_hole circle (at -1.59099 -1.59099 90) (size 0.8 0.8) (drill 0.5) (layers *.Cu *.Mask) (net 42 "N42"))
  (pad 1 thru_hole circle (at -2.25 0 90) (size 0.8 0.8) (drill 0.5) (layers *.Cu *.Mask) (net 42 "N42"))
  (pad 1 thru_hole circle (at -1.59099 1.59099 90) (size 0.8 0.8) (drill 0.5) (layers *.Cu *.Mask) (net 42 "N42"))
  (pad 1 thru_hole circle (at 0 2.25 90) (size 0.8 0.8) (drill 0.5) (layers *.Cu *.Mask) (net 42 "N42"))
  (pad 1 thru_hole circle (at 1.59099 1.59099 90) (size 0.8 0.8) (drill 0.5) (layers *.Cu *.Mask) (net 42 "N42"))
  (pad 1 thru_hole circle (at 2.25 0 90) (size 0.8 0.8) (drill 0.5) (layers *.Cu *.Mask) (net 42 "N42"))
  (pad 1 thru_hole circle (at 0 0 90) (size 6 6) (drill 3) (layers *.Cu *.Mask) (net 42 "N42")))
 (gr_line (start 17.526 22.86) (end 17.526 76.2) (layer Edge.Cuts) (width 0.05))
 (gr_arc (start 26.416 76.2) (end 17.526 76.2) (angle -180) (layer Edge.Cuts) (width 0.05))
 (gr_arc (start 26.416 22.86) (end 35.306 22.86) (angle -180) (layer Edge.Cuts) (width 0.05))
 (gr_line (start 35.306 22.86) (end 35.306 76.2) (layer Edge.Cuts) (width 0.05))
 (segment (start 21.082 25.4) (end 24.13 25.4) (width 1) (layer F.Cu) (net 40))
 (segment (start 33.013 21.773) (end 32.512 21.272) (width 0.2) (layer F.Cu) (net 2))
 (segment (start 33.938 21.773) (end 33.013 21.773) (width 0.2) (layer F.Cu) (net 2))
 (via (at 30.734 23.114) (size 0.8) (drill 0.4) (layers F.Cu B.Cu) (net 2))
 (segment (start 30.693 23.073) (end 30.734 23.114) (width 0.2) (layer F.Cu) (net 2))
 (segment (start 28.038 23.073) (end 30.693 23.073) (width 0.2) (layer F.Cu) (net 2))
 (via (at 32.512 21.082) (size 0.8) (drill 0.4) (layers F.Cu B.Cu) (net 2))
 (segment (start 32.512 21.272) (end 32.512 21.082) (width 0.2) (layer F.Cu) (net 2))
 (segment (start 30.734 23.114) (end 32.004 23.114) (width 0.2) (layer B.Cu) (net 2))
 (segment (start 32.512 22.606) (end 32.512 21.082) (width 0.2) (layer B.Cu) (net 2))
 (segment (start 32.004 23.114) (end 32.512 22.606) (width 0.2) (layer B.Cu) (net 2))
 (segment (start 32.512 19.558) (end 32.258 19.304) (width 0.2) (layer F.Cu) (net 2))
 (segment (start 32.512 21.082) (end 32.512 19.558) (width 0.2) (layer F.Cu) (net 2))
 (segment (start 24.13 38.1) (end 19.05 38.1) (width 1) (layer F.Cu) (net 2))
 (segment (start 25.280001 36.949999) (end 25.280001 24.905999) (width 0.2) (layer F.Cu) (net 2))
 (segment (start 24.13 38.1) (end 25.280001 36.949999) (width 0.2) (layer F.Cu) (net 2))
 (segment (start 25.280001 24.905999) (end 27.113 23.073) (width 0.2) (layer F.Cu) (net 2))
 (segment (start 27.113 23.073) (end 28.038 23.073) (width 0.2) (layer F.Cu) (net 2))
 (segment (start 31.583715 22.271742) (end 31.583715 22.41399) (width 0.2) (layer B.Cu) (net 4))
 (via (at 31.583715 22.41399) (size 0.8) (drill 0.4) (layers F.Cu B.Cu) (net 4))
 (segment (start 33.938 23.073) (end 32.242725 23.073) (width 0.2) (layer F.Cu) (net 4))
 (segment (start 32.242725 23.073) (end 31.583715 22.41399) (width 0.2) (layer F.Cu) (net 4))
 (segment (start 30.05769 21.417719) (end 30.729692 21.417719) (width 0.2) (layer B.Cu) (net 4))
 (segment (start 30.729692 21.417719) (end 31.583715 22.271742) (width 0.2) (layer B.Cu) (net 4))
 (segment (start 25.699998 21.59) (end 29.885409 21.59) (width 0.2) (layer B.Cu) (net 4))
 (segment (start 24.13 33.02) (end 22.86 31.75) (width 0.2) (layer B.Cu) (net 4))
 (segment (start 29.885409 21.59) (end 30.05769 21.417719) (width 0.2) (layer B.Cu) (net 4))
 (segment (start 22.86 24.429998) (end 25.699998 21.59) (width 0.2) (layer B.Cu) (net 4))
 (segment (start 22.86 31.75) (end 22.86 24.429998) (width 0.2) (layer B.Cu) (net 4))
 (segment (start 24.13 33.02) (end 19.05 33.02) (width 1) (layer F.Cu) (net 4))
 (segment (start 25.4 23.876) (end 26.416 22.86) (width 0.2) (layer B.Cu) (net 3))
 (segment (start 26.416 22.86) (end 29.651411 22.86) (width 0.2) (layer B.Cu) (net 3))
 (segment (start 25.4 29.21) (end 25.4 23.876) (width 0.2) (layer B.Cu) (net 3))
 (via (at 30.393691 22.11772) (size 0.8) (drill 0.4) (layers F.Cu B.Cu) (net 3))
 (segment (start 24.13 30.48) (end 25.4 29.21) (width 0.2) (layer B.Cu) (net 3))
 (segment (start 29.651411 22.86) (end 30.393691 22.11772) (width 0.2) (layer B.Cu) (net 3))
 (segment (start 33.938 22.423) (end 32.628727 22.423) (width 0.2) (layer F.Cu) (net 3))
 (segment (start 31.919716 21.713989) (end 30.797422 21.713989) (width 0.2) (layer F.Cu) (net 3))
 (segment (start 30.797422 21.713989) (end 30.393691 22.11772) (width 0.2) (layer F.Cu) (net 3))
 (segment (start 32.628727 22.423) (end 31.919716 21.713989) (width 0.2) (layer F.Cu) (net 3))
 (segment (start 24.13 30.48) (end 21.082 30.48) (width 1) (layer F.Cu) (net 3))
 (segment (start 19.05 27.94) (end 19.05 26.172234) (width 0.2) (layer F.Cu) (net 1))
 (segment (start 19.05 27.94) (end 19.05 23.622) (width 0.2) (layer F.Cu) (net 1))
 (segment (start 20.899 21.773) (end 28.038 21.773) (width 0.2) (layer F.Cu) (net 1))
 (segment (start 19.05 23.622) (end 20.899 21.773) (width 0.2) (layer F.Cu) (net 1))
 (segment (start 30.80801 18.52899) (end 30.508 18.829) (width 0.2) (layer F.Cu) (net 1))
 (segment (start 30.508 18.829) (end 30.508 19.304) (width 0.2) (layer F.Cu) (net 1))
 (segment (start 32.768146 18.52899) (end 30.80801 18.52899) (width 0.2) (layer F.Cu) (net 1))
 (segment (start 33.938 19.698844) (end 32.768146 18.52899) (width 0.2) (layer F.Cu) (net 1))
 (segment (start 33.938 21.123) (end 33.938 19.698844) (width 0.2) (layer F.Cu) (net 1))
 (segment (start 28.038 21.773) (end 29.535 21.773) (width 0.2) (layer F.Cu) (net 1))
 (segment (start 30.508 20.8) (end 30.508 19.304) (width 0.2) (layer F.Cu) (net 1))
 (segment (start 29.535 21.773) (end 30.508 20.8) (width 0.2) (layer F.Cu) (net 1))
 (segment (start 28.038 22.423) (end 29.266 22.423) (width 0.2) (layer F.Cu) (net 1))
 (segment (start 29.535 22.154) (end 29.535 21.773) (width 0.2) (layer F.Cu) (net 1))
 (segment (start 29.266 22.423) (end 29.535 22.154) (width 0.2) (layer F.Cu) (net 1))
 (segment (start 28.038 21.123) (end 29.378 21.123) (width 0.2) (layer F.Cu) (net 1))
 (segment (start 29.535 21.28) (end 29.535 21.773) (width 0.2) (layer F.Cu) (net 1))
 (segment (start 29.378 21.123) (end 29.535 21.28) (width 0.2) (layer F.Cu) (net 1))
 (segment (start 24.13 27.94) (end 19.05 27.94) (width 1) (layer F.Cu) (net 1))
 (segment (start 31.75 30.48) (end 26.67 30.48) (width 1) (layer F.Cu) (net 39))
 (segment (start 24.13 35.56) (end 21.082 35.56) (width 1) (layer F.Cu) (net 38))
 (segment (start 26.67 38.1) (end 29.718 38.1) (width 1) (layer F.Cu) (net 37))
 (segment (start 24.13 45.72) (end 21.082 45.72) (width 1) (layer F.Cu) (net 34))
 (segment (start 26.67 45.72) (end 31.75 45.72) (width 1) (layer F.Cu) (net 33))
 (segment (start 24.13 53.34) (end 19.05 53.34) (width 1) (layer F.Cu) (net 30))
 (segment (start 26.67 53.34) (end 30.226 53.34) (width 1) (layer F.Cu) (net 29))
 (segment (start 24.13 60.96) (end 21.082 60.96) (width 1) (layer F.Cu) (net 26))
 (segment (start 24.13 63.5) (end 19.05 63.5) (width 1) (layer F.Cu) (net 24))
 (segment (start 24.13 66.04) (end 21.082 66.04) (width 1) (layer F.Cu) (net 23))
 (segment (start 24.13 68.58) (end 19.05 68.58) (width 1) (layer F.Cu) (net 22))
 (segment (start 24.13 71.12) (end 21.082 71.12) (width 1) (layer F.Cu) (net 20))
 (segment (start 24.13 73.66) (end 19.05 73.66) (width 1) (layer F.Cu) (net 19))
 (segment (start 26.67 25.4) (end 33.782 25.4) (width 1) (layer F.Cu) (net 17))
 (segment (start 33.782 27.94) (end 26.67 27.94) (width 1) (layer F.Cu) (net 18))
 (segment (start 26.67 33.02) (end 33.782 33.02) (width 1) (layer F.Cu) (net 15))
 (segment (start 26.67 35.56) (end 33.782 35.56) (width 1) (layer F.Cu) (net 16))
 (segment (start 33.782 40.64) (end 31.75 40.64) (width 1) (layer F.Cu) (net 13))
 (segment (start 33.782 40.64) (end 26.67 40.64) (width 1) (layer F.Cu) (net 13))
 (segment (start 33.782 43.18) (end 29.718 43.18) (width 1) (layer F.Cu) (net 14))
 (segment (start 26.67 43.18) (end 29.718 43.18) (width 1) (layer F.Cu) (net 14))
 (segment (start 26.67 48.26) (end 33.782 48.26) (width 1) (layer F.Cu) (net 11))
 (segment (start 26.67 50.8) (end 33.782 50.8) (width 1) (layer F.Cu) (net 12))
 (segment (start 26.67 55.88) (end 33.782 55.88) (width 1) (layer F.Cu) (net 9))
 (segment (start 26.67 58.42) (end 33.782 58.42) (width 1) (layer F.Cu) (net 10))
 (segment (start 26.67 63.5) (end 33.782 63.5) (width 1) (layer F.Cu) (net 7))
 (segment (start 26.67 66.04) (end 33.782 66.04) (width 1) (layer F.Cu) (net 8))
 (segment (start 26.67 71.12) (end 33.782 71.12) (width 1) (layer F.Cu) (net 5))
 (segment (start 26.67 73.66) (end 33.782 73.66) (width 1) (layer F.Cu) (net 6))
 (segment (start 24.13 40.64) (end 21.082 40.64) (width 1) (layer F.Cu) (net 36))
 (segment (start 24.13 43.18) (end 19.05 43.18) (width 1) (layer F.Cu) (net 35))
 (segment (start 24.13 48.26) (end 19.05 48.26) (width 1) (layer F.Cu) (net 32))
 (segment (start 24.13 50.8) (end 21.082 50.8) (width 1) (layer F.Cu) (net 31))
 (segment (start 24.13 55.88) (end 21.082 55.88) (width 1) (layer F.Cu) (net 28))
 (segment (start 24.13 58.42) (end 19.05 58.42) (width 1) (layer F.Cu) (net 27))
 (segment (start 26.67 60.96) (end 31.75 60.96) (width 1) (layer F.Cu) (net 25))
 (segment (start 26.67 68.58) (end 29.718 68.58) (width 1) (layer F.Cu) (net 21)))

